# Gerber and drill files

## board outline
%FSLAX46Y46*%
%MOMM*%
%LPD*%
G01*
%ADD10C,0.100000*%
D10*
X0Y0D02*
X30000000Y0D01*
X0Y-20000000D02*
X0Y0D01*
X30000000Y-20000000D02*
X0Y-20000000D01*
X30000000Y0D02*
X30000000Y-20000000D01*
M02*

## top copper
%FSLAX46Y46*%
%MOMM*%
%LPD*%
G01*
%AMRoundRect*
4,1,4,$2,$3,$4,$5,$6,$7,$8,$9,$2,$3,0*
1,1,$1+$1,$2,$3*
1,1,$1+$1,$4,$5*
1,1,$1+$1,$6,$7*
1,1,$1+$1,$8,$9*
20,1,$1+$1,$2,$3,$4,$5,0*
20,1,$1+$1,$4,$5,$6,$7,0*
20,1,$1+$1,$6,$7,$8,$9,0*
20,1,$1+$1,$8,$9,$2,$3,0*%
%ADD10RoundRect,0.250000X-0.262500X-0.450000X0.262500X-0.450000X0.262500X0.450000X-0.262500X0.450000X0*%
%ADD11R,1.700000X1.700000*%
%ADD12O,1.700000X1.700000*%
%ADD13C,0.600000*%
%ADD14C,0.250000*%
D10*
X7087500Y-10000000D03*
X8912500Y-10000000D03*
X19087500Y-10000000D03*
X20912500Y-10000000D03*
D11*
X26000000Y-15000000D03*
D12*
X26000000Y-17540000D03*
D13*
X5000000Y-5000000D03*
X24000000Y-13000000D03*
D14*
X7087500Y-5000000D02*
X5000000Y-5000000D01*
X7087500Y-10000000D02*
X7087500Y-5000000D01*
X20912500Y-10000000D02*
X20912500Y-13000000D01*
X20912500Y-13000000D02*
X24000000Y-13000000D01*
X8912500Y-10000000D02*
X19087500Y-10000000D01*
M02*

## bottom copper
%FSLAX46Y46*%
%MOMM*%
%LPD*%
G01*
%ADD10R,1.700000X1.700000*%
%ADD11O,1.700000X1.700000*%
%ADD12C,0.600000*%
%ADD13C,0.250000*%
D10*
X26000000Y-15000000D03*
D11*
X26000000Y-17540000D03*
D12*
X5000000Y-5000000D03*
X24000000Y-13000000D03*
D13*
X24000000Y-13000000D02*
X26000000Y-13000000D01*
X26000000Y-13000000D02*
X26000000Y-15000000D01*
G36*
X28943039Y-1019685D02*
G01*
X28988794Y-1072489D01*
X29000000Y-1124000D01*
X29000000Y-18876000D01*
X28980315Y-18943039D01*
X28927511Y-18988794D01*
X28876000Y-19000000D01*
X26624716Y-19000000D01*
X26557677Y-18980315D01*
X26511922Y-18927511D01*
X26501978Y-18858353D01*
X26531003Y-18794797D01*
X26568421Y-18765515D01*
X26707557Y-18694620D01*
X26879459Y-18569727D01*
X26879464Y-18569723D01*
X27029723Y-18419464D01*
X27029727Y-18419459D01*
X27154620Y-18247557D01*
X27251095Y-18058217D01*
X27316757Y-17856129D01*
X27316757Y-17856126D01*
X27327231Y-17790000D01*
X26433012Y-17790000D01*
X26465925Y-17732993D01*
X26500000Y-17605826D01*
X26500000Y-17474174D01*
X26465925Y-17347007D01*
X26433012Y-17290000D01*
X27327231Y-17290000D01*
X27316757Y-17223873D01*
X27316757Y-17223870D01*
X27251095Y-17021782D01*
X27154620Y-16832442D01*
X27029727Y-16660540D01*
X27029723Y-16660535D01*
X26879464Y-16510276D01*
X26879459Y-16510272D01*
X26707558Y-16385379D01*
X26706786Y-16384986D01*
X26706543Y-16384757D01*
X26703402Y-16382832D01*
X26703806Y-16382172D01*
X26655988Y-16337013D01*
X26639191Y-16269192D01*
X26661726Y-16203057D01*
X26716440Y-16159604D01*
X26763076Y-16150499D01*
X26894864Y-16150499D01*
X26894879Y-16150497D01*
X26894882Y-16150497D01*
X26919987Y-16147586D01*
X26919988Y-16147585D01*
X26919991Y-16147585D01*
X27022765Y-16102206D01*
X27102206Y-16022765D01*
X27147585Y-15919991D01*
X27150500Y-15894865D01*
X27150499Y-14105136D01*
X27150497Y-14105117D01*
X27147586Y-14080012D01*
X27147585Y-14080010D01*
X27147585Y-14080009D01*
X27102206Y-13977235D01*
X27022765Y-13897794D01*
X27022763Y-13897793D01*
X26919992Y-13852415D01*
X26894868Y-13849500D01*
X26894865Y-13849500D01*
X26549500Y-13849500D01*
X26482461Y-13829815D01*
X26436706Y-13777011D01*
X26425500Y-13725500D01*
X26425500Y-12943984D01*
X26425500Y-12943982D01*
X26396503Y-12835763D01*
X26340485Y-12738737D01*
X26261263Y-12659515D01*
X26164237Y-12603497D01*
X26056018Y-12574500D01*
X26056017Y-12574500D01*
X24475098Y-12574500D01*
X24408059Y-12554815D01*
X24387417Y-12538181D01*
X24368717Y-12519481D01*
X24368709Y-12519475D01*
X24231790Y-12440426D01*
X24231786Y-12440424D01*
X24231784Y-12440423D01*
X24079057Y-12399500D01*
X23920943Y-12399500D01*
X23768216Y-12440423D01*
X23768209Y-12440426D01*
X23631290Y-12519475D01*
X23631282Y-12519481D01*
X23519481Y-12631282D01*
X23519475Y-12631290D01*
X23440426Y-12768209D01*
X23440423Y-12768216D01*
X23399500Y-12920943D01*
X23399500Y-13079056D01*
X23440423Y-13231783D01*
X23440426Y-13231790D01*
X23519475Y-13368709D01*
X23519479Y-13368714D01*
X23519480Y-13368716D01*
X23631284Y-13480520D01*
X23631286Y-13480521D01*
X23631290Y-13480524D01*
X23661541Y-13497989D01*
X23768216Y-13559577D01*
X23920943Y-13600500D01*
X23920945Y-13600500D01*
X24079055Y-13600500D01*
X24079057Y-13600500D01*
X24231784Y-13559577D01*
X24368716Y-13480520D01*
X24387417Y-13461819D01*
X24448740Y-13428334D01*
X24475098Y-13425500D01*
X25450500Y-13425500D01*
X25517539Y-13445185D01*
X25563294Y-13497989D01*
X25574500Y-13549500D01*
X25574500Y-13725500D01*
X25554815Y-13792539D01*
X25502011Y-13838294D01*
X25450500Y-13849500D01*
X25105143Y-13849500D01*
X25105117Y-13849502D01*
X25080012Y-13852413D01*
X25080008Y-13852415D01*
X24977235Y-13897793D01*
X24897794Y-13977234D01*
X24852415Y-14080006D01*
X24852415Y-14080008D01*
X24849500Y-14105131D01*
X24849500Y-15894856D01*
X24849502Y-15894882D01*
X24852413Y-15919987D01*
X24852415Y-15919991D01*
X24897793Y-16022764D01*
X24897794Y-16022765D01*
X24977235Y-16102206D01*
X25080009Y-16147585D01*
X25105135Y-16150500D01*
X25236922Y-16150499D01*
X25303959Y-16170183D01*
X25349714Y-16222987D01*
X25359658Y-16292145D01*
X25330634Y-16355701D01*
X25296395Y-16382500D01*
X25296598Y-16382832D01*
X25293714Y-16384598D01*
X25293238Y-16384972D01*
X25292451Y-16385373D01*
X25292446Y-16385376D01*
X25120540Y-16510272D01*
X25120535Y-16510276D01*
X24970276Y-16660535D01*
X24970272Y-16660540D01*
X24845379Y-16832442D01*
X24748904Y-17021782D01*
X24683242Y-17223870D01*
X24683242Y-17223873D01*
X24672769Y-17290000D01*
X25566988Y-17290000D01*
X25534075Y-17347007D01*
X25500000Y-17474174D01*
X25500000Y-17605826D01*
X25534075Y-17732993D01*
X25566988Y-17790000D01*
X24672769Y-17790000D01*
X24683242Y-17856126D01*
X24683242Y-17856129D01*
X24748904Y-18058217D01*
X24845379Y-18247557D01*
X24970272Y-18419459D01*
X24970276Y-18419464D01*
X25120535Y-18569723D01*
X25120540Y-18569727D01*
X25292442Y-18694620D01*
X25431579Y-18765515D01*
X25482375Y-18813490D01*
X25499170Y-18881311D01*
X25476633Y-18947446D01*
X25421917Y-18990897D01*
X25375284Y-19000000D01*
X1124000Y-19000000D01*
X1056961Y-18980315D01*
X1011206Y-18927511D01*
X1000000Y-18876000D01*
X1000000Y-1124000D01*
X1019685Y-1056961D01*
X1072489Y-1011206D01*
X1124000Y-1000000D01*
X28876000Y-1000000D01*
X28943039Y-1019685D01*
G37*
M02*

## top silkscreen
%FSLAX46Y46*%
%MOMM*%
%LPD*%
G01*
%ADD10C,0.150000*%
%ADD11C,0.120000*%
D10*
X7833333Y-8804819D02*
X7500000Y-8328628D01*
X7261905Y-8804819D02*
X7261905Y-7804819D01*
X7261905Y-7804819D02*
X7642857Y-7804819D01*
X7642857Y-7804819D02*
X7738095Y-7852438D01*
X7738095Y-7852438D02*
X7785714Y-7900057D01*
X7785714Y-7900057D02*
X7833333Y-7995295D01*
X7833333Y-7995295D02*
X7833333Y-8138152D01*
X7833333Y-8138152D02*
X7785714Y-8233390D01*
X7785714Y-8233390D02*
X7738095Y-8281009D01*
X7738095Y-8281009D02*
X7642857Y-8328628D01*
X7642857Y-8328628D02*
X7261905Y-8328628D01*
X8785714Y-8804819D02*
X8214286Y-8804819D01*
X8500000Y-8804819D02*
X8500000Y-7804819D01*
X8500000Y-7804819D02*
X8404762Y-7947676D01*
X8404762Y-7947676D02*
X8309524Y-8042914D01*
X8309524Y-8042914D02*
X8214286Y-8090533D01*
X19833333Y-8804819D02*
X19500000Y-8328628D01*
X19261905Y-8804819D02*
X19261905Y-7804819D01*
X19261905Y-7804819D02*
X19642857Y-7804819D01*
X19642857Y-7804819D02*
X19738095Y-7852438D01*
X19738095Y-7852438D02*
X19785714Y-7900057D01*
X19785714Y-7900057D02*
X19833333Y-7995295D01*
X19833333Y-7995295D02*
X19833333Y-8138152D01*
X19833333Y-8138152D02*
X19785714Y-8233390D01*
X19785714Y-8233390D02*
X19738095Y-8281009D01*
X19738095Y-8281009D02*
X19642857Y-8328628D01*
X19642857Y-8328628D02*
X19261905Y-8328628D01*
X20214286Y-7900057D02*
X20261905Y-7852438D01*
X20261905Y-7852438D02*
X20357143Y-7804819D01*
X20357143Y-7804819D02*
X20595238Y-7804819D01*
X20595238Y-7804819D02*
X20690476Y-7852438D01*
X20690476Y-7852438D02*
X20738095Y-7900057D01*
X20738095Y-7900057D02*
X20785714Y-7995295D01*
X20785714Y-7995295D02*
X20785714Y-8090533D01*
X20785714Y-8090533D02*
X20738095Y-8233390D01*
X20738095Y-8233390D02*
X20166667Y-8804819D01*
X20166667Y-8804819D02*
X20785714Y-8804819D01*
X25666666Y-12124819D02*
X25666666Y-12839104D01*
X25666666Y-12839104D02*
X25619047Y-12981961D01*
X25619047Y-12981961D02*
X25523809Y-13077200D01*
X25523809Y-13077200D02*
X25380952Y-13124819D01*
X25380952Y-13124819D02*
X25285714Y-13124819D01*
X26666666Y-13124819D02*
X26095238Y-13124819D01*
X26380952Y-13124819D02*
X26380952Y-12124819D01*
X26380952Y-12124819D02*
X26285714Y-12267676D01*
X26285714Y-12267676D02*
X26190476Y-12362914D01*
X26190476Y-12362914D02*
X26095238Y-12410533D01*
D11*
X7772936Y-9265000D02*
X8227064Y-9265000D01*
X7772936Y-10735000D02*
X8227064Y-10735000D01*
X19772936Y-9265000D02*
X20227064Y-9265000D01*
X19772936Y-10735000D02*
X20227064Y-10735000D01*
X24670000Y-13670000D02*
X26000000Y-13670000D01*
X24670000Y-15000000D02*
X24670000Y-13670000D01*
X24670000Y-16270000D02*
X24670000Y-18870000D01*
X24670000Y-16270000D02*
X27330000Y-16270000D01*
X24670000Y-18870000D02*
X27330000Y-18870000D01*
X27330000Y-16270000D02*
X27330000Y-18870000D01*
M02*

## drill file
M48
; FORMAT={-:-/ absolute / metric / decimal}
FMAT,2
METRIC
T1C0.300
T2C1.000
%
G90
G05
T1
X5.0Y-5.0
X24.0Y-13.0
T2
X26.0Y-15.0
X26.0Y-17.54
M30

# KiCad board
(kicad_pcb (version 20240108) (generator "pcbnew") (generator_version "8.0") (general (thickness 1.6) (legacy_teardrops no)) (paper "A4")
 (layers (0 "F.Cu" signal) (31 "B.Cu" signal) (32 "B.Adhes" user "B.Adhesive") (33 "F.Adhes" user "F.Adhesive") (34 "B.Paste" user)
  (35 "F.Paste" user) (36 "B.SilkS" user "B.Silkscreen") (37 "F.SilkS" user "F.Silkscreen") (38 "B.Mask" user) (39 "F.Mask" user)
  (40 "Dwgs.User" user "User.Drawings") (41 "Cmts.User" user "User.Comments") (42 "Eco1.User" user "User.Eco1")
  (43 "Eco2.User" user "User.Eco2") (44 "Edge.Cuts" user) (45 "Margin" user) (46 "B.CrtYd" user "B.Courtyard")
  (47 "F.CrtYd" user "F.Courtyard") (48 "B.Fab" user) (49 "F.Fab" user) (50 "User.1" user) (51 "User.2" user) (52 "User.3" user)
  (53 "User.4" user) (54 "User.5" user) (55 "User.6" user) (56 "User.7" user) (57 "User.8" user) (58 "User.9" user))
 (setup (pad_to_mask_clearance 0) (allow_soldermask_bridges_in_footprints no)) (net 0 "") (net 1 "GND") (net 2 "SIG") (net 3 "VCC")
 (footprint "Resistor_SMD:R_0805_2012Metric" (layer "F.Cu") (at 8 10)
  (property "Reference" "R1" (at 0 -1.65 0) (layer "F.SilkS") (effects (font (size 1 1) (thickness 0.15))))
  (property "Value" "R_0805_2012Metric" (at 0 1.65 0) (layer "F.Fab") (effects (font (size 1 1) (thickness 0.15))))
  (fp_line (start -0.227064 -0.735) (end 0.227064 -0.735) (stroke (width 0.12) (type solid)) (layer "F.SilkS"))
  (fp_line (start -0.227064 0.735) (end 0.227064 0.735) (stroke (width 0.12) (type solid)) (layer "F.SilkS"))
  (pad "1" smd roundrect (at -0.9125 0) (size 1.025 1.4) (layers "F.Cu" "F.Paste" "F.Mask") (roundrect_rratio 0.243902) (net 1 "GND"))
  (pad "2" smd roundrect (at 0.9125 0) (size 1.025 1.4) (layers "F.Cu" "F.Paste" "F.Mask") (roundrect_rratio 0.243902) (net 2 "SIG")))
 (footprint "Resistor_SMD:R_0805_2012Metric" (layer "F.Cu") (at 20 10)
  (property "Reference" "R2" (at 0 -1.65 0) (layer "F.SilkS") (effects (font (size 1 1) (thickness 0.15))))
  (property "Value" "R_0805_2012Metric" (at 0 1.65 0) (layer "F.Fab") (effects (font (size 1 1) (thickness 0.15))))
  (fp_line (start -0.227064 -0.735) (end 0.227064 -0.735) (stroke (width 0.12) (type solid)) (layer "F.SilkS"))
  (fp_line (start -0.227064 0.735) (end 0.227064 0.735) (stroke (width 0.12) (type solid)) (layer "F.SilkS"))
  (pad "1" smd roundrect (at -0.9125 0) (size 1.025 1.4) (layers "F.Cu" "F.Paste" "F.Mask") (roundrect_rratio 0.243902) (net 2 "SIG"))
  (pad "2" smd roundrect (at 0.9125 0) (size 1.025 1.4) (layers "F.Cu" "F.Paste" "F.Mask") (roundrect_rratio 0.243902) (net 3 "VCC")))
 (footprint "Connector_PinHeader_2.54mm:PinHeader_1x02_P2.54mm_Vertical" (layer "F.Cu") (at 26 15)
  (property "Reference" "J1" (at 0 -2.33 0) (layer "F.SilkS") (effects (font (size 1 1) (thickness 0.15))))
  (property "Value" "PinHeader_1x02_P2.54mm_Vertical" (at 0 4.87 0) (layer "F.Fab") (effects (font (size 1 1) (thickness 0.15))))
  (fp_line (start -1.33 -1.33) (end 0 -1.33) (stroke (width 0.12) (type solid)) (layer "F.SilkS"))
  (fp_line (start -1.33 0) (end -1.33 -1.33) (stroke (width 0.12) (type solid)) (layer "F.SilkS"))
  (fp_line (start -1.33 1.27) (end -1.33 3.87) (stroke (width 0.12) (type solid)) (layer "F.SilkS"))
  (fp_line (start -1.33 1.27) (end 1.33 1.27) (stroke (width 0.12) (type solid)) (layer "F.SilkS"))
  (fp_line (start -1.33 3.87) (end 1.33 3.87) (stroke (width 0.12) (type solid)) (layer "F.SilkS"))
  (fp_line (start 1.33 1.27) (end 1.33 3.87) (stroke (width 0.12) (type solid)) (layer "F.SilkS"))
  (pad "1" thru_hole rect (at 0 0) (size 1.7 1.7) (drill 1) (layers "*.Cu" "*.Mask") (remove_unused_layers no) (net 3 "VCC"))
  (pad "2" thru_hole oval (at 0 2.54) (size 1.7 1.7) (drill 1) (layers "*.Cu" "*.Mask") (remove_unused_layers no) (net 1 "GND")))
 (gr_line (start 0 0) (end 30 0) (stroke (width 0.1) (type default)) (layer "Edge.Cuts"))
 (gr_line (start 0 20) (end 0 0) (stroke (width 0.1) (type default)) (layer "Edge.Cuts"))
 (gr_line (start 30 20) (end 0 20) (stroke (width 0.1) (type default)) (layer "Edge.Cuts"))
 (gr_line (start 30 0) (end 30 20) (stroke (width 0.1) (type default)) (layer "Edge.Cuts"))
 (segment (start 7.0875 5) (end 5 5) (width 0.25) (layer "F.Cu") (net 1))
 (segment (start 7.0875 10) (end 7.0875 5) (width 0.25) (layer "F.Cu") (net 1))
 (via (at 5 5) (size 0.6) (drill 0.3) (layers "F.Cu" "B.Cu") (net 1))
 (segment (start 20.9125 10) (end 20.9125 13) (width 0.25) (layer "F.Cu") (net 3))
 (segment (start 20.9125 13) (end 24 13) (width 0.25) (layer "F.Cu") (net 3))
 (via (at 24 13) (size 0.6) (drill 0.3) (layers "F.Cu" "B.Cu") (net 3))
 (segment (start 24 13) (end 26 13) (width 0.25) (layer "B.Cu") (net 3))
 (segment (start 26 13) (end 26 15) (width 0.25) (layer "B.Cu") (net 3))
 (segment (start 8.9125 10) (end 19.0875 10) (width 0.25) (layer "F.Cu") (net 2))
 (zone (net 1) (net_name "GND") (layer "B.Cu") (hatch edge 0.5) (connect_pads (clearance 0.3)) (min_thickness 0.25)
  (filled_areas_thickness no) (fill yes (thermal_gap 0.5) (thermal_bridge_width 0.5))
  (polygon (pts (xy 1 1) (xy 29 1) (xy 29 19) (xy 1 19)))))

